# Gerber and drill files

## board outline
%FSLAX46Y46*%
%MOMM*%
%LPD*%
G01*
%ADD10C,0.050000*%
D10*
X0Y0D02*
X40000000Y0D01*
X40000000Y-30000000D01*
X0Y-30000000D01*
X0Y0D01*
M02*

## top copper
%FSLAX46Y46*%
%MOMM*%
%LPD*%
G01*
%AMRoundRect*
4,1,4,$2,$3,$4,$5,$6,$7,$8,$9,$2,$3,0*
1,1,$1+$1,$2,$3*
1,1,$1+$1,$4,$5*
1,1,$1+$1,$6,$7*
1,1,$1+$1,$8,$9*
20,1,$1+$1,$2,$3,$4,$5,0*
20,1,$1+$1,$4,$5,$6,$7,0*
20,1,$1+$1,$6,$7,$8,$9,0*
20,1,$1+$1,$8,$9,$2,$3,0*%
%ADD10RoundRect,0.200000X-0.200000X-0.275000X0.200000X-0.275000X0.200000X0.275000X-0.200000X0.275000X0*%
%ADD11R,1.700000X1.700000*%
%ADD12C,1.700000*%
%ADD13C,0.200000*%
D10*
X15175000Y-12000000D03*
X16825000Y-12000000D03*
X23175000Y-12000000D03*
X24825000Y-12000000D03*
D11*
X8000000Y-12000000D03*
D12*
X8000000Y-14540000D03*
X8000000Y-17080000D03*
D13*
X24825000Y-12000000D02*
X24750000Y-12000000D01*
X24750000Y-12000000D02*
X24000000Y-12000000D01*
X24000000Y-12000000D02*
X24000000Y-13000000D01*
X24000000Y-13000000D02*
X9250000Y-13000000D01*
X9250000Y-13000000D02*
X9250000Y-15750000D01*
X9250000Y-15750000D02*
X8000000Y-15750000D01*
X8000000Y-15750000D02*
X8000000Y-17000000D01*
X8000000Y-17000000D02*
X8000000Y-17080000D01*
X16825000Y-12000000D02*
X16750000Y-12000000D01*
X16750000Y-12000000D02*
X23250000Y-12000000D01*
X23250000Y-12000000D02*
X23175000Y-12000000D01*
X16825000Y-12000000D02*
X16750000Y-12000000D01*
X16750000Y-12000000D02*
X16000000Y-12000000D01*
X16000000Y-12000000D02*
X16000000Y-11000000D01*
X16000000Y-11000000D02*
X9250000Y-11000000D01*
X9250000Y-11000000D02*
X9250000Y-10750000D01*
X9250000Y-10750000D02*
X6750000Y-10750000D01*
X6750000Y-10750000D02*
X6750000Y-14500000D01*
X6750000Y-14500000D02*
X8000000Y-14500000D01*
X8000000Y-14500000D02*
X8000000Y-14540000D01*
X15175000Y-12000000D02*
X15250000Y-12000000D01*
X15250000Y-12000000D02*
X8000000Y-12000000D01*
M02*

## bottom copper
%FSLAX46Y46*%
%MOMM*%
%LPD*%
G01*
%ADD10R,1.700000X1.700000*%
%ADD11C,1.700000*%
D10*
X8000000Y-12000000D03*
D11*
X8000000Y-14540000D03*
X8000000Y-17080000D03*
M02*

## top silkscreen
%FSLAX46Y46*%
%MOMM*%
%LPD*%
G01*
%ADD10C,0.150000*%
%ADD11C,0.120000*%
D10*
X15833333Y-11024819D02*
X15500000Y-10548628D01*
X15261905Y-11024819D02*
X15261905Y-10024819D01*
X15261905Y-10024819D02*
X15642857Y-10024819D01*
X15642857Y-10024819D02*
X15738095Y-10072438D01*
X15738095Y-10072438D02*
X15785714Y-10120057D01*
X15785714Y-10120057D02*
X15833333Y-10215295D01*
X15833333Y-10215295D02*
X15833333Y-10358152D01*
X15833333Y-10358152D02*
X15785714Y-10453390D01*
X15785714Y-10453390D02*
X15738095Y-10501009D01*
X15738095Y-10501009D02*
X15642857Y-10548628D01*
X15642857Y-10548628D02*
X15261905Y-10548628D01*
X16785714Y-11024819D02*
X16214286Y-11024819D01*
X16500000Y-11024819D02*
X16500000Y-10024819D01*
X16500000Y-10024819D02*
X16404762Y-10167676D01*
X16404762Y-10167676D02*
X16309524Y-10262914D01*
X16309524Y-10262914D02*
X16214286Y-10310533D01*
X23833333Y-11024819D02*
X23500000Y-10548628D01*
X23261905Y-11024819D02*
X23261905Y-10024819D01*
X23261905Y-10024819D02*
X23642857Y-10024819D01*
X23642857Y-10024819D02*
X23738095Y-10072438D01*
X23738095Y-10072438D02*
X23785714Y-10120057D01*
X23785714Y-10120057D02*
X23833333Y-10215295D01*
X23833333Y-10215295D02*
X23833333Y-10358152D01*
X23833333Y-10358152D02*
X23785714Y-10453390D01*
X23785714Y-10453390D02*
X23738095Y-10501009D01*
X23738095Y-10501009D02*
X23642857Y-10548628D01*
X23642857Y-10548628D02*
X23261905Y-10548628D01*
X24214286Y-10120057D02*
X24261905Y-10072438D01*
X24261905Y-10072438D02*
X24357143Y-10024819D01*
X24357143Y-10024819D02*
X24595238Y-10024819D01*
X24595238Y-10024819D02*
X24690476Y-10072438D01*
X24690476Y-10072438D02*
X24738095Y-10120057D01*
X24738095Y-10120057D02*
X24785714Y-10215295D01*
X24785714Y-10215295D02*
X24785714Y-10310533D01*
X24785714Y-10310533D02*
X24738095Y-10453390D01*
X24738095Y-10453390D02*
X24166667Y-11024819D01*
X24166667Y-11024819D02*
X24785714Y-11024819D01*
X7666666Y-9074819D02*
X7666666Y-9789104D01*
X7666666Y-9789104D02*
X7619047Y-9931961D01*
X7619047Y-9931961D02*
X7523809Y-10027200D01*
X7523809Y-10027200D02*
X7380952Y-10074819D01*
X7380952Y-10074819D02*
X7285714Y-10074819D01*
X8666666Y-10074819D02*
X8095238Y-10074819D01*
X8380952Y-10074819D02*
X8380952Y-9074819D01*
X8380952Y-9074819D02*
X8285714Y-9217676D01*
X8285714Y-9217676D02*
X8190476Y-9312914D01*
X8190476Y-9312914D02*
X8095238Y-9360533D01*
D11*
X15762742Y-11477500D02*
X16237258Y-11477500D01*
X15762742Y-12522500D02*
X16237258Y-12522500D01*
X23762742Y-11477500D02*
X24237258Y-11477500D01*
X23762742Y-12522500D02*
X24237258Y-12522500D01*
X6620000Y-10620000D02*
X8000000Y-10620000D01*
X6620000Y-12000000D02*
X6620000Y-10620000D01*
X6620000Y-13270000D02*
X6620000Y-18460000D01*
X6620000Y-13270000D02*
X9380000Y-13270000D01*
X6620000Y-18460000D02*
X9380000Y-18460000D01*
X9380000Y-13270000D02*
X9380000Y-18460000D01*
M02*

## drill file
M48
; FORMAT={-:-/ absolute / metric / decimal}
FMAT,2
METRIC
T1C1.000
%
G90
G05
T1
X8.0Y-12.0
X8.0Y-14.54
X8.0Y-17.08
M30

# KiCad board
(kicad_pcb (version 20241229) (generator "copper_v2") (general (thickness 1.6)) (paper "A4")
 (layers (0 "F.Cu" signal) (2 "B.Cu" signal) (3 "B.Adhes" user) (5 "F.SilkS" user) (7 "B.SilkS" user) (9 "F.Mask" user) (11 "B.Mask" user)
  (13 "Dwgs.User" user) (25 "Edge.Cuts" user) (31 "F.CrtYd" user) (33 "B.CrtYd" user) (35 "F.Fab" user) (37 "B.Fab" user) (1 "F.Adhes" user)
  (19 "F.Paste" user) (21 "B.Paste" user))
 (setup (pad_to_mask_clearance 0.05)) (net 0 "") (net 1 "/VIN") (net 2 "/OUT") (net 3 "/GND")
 (gr_rect (start 0 0) (end 40 30) (stroke (width .05) (type default)) (fill none) (layer "Edge.Cuts"))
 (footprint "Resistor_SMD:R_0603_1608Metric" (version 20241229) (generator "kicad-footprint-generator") (layer "F.Cu")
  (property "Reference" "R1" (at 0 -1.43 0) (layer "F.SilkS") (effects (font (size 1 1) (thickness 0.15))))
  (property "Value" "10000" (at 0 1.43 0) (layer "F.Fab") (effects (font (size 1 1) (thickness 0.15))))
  (fp_line (start -0.237258 -0.5225) (end 0.237258 -0.5225) (stroke (width 0.12) (type solid)) (layer "F.SilkS"))
  (fp_line (start -0.237258 0.5225) (end 0.237258 0.5225) (stroke (width 0.12) (type solid)) (layer "F.SilkS"))
  (pad "1" smd roundrect (at -0.825 0) (size 0.8 0.95) (layers "F.Cu" "F.Mask" "F.Paste") (roundrect_rratio 0.25) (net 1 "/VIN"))
  (pad "2" smd roundrect (at 0.825 0) (size 0.8 0.95) (layers "F.Cu" "F.Mask" "F.Paste") (roundrect_rratio 0.25) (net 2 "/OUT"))
  (at 16 12 0))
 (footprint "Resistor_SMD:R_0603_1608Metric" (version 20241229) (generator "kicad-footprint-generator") (layer "F.Cu")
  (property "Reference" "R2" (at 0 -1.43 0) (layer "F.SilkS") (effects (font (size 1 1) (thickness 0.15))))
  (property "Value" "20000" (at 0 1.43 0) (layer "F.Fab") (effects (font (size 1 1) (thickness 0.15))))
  (fp_line (start -0.237258 -0.5225) (end 0.237258 -0.5225) (stroke (width 0.12) (type solid)) (layer "F.SilkS"))
  (fp_line (start -0.237258 0.5225) (end 0.237258 0.5225) (stroke (width 0.12) (type solid)) (layer "F.SilkS"))
  (pad "1" smd roundrect (at -0.825 0) (size 0.8 0.95) (layers "F.Cu" "F.Mask" "F.Paste") (roundrect_rratio 0.25) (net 2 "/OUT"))
  (pad "2" smd roundrect (at 0.825 0) (size 0.8 0.95) (layers "F.Cu" "F.Mask" "F.Paste") (roundrect_rratio 0.25) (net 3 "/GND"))
  (at 24 12 0))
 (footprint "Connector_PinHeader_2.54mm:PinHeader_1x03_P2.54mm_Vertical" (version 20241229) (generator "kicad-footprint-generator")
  (layer "F.Cu")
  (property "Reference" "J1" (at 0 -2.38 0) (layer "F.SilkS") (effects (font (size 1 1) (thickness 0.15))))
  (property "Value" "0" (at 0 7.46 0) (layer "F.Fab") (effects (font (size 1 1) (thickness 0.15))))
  (fp_line (start -1.38 -1.38) (end 0 -1.38) (stroke (width 0.12) (type solid)) (layer "F.SilkS"))
  (fp_line (start -1.38 0) (end -1.38 -1.38) (stroke (width 0.12) (type solid)) (layer "F.SilkS"))
  (fp_line (start -1.38 1.27) (end -1.38 6.46) (stroke (width 0.12) (type solid)) (layer "F.SilkS"))
  (fp_line (start -1.38 1.27) (end 1.38 1.27) (stroke (width 0.12) (type solid)) (layer "F.SilkS"))
  (fp_line (start -1.38 6.46) (end 1.38 6.46) (stroke (width 0.12) (type solid)) (layer "F.SilkS"))
  (fp_line (start 1.38 1.27) (end 1.38 6.46) (stroke (width 0.12) (type solid)) (layer "F.SilkS"))
  (pad "1" thru_hole rect (at 0 0) (size 1.7 1.7) (drill 1) (layers "*.Cu" "*.Mask") (remove_unused_layers no) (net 1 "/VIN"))
  (pad "2" thru_hole circle (at 0 2.54) (size 1.7 1.7) (drill 1) (layers "*.Cu" "*.Mask") (remove_unused_layers no) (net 2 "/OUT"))
  (pad "3" thru_hole circle (at 0 5.08) (size 1.7 1.7) (drill 1) (layers "*.Cu" "*.Mask") (remove_unused_layers no) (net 3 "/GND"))
  (at 8 12 0))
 (segment (start 24.825 12) (end 24.75 12) (width 0.2) (layer "F.Cu") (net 3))
 (segment (start 24.75 12) (end 24 12) (width 0.2) (layer "F.Cu") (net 3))
 (segment (start 24 12) (end 24 13) (width 0.2) (layer "F.Cu") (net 3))
 (segment (start 24 13) (end 9.25 13) (width 0.2) (layer "F.Cu") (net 3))
 (segment (start 9.25 13) (end 9.25 15.75) (width 0.2) (layer "F.Cu") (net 3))
 (segment (start 9.25 15.75) (end 8 15.75) (width 0.2) (layer "F.Cu") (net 3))
 (segment (start 8 15.75) (end 8 17) (width 0.2) (layer "F.Cu") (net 3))
 (segment (start 8 17) (end 8 17.08) (width 0.2) (layer "F.Cu") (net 3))
 (segment (start 16.825 12) (end 16.75 12) (width 0.2) (layer "F.Cu") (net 2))
 (segment (start 16.75 12) (end 23.25 12) (width 0.2) (layer "F.Cu") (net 2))
 (segment (start 23.25 12) (end 23.175 12) (width 0.2) (layer "F.Cu") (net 2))
 (segment (start 16.825 12) (end 16.75 12) (width 0.2) (layer "F.Cu") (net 2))
 (segment (start 16.75 12) (end 16 12) (width 0.2) (layer "F.Cu") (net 2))
 (segment (start 16 12) (end 16 11) (width 0.2) (layer "F.Cu") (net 2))
 (segment (start 16 11) (end 9.25 11) (width 0.2) (layer "F.Cu") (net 2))
 (segment (start 9.25 11) (end 9.25 10.75) (width 0.2) (layer "F.Cu") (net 2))
 (segment (start 9.25 10.75) (end 6.75 10.75) (width 0.2) (layer "F.Cu") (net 2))
 (segment (start 6.75 10.75) (end 6.75 14.5) (width 0.2) (layer "F.Cu") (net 2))
 (segment (start 6.75 14.5) (end 8 14.5) (width 0.2) (layer "F.Cu") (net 2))
 (segment (start 8 14.5) (end 8 14.54) (width 0.2) (layer "F.Cu") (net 2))
 (segment (start 15.175 12) (end 15.25 12) (width 0.2) (layer "F.Cu") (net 1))
 (segment (start 15.25 12) (end 8 12) (width 0.2) (layer "F.Cu") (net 1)))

